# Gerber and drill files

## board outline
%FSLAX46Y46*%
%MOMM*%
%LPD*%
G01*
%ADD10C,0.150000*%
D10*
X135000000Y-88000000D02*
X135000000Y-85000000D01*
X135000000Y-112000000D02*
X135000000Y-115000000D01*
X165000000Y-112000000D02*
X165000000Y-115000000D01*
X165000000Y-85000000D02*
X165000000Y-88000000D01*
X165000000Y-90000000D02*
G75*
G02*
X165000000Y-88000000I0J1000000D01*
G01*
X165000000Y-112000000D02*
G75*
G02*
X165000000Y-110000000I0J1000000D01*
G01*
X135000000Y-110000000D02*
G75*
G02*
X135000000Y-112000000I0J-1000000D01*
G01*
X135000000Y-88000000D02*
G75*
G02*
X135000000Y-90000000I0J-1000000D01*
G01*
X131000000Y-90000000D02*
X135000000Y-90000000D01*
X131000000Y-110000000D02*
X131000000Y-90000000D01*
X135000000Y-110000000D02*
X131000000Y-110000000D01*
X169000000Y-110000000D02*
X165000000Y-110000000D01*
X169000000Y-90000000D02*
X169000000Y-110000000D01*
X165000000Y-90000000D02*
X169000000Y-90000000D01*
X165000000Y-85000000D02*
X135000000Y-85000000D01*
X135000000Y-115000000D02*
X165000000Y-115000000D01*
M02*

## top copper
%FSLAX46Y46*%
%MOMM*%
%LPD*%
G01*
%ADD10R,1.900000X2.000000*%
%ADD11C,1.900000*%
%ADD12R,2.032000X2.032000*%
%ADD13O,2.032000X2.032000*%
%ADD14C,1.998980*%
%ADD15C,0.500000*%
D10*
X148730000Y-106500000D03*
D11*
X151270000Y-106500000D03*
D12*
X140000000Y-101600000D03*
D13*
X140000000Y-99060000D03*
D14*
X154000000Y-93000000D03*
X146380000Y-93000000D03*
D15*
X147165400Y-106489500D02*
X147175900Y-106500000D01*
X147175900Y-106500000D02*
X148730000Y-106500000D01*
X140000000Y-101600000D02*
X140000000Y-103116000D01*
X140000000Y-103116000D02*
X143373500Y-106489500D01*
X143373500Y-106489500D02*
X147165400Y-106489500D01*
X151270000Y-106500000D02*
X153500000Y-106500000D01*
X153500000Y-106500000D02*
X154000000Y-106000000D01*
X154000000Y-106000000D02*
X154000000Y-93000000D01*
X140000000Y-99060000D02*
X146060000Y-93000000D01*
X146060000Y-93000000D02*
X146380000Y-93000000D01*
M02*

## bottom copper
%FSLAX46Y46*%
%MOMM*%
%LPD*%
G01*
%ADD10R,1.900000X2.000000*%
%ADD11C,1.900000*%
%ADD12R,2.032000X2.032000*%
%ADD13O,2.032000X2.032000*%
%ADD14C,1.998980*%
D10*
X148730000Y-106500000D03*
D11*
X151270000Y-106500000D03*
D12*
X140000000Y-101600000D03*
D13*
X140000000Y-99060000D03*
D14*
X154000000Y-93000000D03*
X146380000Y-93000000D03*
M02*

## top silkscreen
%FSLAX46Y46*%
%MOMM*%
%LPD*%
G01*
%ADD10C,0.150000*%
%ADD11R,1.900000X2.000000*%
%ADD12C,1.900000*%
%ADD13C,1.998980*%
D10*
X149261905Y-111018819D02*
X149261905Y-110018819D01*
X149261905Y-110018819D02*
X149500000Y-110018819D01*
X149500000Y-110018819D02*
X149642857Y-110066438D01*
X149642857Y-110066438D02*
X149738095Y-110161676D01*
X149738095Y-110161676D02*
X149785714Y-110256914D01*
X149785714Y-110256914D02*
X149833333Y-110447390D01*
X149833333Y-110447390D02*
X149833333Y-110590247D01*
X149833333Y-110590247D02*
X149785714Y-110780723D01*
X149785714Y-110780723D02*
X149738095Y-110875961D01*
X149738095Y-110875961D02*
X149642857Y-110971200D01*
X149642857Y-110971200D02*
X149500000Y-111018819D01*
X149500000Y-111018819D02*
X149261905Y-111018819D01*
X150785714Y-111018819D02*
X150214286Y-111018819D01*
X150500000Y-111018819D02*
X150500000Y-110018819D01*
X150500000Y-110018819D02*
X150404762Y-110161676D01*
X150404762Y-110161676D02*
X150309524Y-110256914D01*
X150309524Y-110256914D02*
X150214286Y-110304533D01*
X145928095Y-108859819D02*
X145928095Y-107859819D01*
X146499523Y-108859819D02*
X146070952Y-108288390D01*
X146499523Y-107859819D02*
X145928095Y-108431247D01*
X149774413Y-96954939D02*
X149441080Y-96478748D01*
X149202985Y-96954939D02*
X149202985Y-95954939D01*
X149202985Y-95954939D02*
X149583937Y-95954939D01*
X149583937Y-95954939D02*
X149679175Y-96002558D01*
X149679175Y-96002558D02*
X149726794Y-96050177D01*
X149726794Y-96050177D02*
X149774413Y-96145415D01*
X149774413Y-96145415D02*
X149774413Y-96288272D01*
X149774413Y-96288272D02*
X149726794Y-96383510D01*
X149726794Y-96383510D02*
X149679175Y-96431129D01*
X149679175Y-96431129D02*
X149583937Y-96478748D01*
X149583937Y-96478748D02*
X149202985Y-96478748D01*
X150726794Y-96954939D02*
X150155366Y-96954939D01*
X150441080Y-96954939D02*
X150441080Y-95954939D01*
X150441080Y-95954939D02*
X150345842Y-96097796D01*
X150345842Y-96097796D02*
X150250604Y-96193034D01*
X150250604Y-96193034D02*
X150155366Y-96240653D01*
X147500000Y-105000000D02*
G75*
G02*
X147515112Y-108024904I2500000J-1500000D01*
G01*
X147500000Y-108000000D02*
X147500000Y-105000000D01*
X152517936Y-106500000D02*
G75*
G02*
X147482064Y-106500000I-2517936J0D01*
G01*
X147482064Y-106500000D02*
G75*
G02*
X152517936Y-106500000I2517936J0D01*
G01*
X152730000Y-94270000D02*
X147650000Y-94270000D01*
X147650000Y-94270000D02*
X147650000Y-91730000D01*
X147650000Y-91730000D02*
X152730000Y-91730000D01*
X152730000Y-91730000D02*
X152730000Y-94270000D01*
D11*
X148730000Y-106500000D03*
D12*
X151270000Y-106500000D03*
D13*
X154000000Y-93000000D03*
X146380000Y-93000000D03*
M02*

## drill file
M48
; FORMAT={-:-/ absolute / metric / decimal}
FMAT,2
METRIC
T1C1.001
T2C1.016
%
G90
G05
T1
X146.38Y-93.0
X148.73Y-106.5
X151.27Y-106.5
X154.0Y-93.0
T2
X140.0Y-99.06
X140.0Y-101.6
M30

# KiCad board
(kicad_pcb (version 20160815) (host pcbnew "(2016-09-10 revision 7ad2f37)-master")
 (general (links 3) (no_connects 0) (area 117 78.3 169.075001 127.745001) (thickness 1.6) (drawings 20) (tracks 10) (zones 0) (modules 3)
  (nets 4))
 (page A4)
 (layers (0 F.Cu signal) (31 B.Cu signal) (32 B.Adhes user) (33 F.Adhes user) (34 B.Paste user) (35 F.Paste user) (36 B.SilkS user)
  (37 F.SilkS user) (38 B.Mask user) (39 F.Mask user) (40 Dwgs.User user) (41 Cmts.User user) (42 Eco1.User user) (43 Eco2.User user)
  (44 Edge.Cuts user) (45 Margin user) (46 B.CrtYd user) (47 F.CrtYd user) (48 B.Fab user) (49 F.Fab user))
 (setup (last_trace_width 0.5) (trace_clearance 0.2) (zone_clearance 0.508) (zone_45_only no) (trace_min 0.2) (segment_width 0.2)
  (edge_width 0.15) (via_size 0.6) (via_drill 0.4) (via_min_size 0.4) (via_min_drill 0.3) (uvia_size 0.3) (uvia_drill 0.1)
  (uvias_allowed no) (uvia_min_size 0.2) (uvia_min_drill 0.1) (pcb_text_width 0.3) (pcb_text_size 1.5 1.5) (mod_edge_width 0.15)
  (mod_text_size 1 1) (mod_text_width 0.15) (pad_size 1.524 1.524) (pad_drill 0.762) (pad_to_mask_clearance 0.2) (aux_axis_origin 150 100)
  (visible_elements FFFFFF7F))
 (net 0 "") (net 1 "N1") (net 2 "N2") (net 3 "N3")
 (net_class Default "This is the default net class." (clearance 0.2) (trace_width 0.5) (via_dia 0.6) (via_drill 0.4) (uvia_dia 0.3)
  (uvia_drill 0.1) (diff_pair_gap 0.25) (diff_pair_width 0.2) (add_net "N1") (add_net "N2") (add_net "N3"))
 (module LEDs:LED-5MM (layer F.Cu) (at 150 106.5)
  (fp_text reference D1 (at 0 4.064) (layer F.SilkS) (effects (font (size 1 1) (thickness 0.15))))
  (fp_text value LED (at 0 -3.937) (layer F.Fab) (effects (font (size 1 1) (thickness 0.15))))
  (fp_arc (start 0 0) (end -2.5 -1.5) (angle 297.5) (layer F.SilkS) (width 0.15))
  (fp_line (start -2.5 1.5) (end -2.5 -1.5) (layer F.SilkS) (width 0.15))
  (fp_circle (center 0 0) (end -0.3 -2.5) (layer F.SilkS) (width 0.15))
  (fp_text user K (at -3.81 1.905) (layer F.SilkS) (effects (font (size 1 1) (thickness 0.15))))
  (pad 1 thru_hole rect (at -1.27 0 90) (size 2 1.9) (drill 1.00076) (layers *.Cu *.Mask F.SilkS) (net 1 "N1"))
  (pad 2 thru_hole circle (at 1.27 0) (size 1.9 1.9) (drill 1.00076) (layers *.Cu *.Mask F.SilkS) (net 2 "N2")))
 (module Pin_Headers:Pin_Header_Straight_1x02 (layer B.Cu) (at 140 101.6)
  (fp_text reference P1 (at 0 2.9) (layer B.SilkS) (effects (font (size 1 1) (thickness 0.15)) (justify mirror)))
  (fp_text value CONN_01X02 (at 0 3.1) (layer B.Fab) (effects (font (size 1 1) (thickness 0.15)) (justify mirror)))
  (pad 1 thru_hole rect (at 0 0) (size 2.032 2.032) (drill 1.016) (layers *.Cu *.Mask B.SilkS) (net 1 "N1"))
  (pad 2 thru_hole oval (at 0 -2.54) (size 2.032 2.032) (drill 1.016) (layers *.Cu *.Mask B.SilkS) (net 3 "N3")))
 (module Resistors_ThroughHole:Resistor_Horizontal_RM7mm (layer F.Cu) (at 154 93 180)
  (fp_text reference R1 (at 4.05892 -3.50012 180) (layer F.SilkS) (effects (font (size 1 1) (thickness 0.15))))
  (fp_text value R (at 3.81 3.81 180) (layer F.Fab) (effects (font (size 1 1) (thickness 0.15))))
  (fp_line (start 1.27 -1.27) (end 6.35 -1.27) (layer F.SilkS) (width 0.15))
  (fp_line (start 6.35 -1.27) (end 6.35 1.27) (layer F.SilkS) (width 0.15))
  (fp_line (start 6.35 1.27) (end 1.27 1.27) (layer F.SilkS) (width 0.15))
  (fp_line (start 1.27 1.27) (end 1.27 -1.27) (layer F.SilkS) (width 0.15))
  (pad 1 thru_hole circle (at 0 0 180) (size 1.99898 1.99898) (drill 1.00076) (layers *.Cu *.SilkS *.Mask) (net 2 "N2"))
  (pad 2 thru_hole circle (at 7.62 0 180) (size 1.99898 1.99898) (drill 1.00076) (layers *.Cu *.SilkS *.Mask) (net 3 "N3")))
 (gr_line (start 135 88) (end 135 85) (layer Edge.Cuts) (width 0.15))
 (gr_line (start 135 112) (end 135 115) (layer Edge.Cuts) (width 0.15))
 (gr_line (start 165 112) (end 165 115) (layer Edge.Cuts) (width 0.15))
 (gr_line (start 165 85) (end 165 88) (layer Edge.Cuts) (width 0.15))
 (gr_arc (start 165 89) (end 165 90) (angle 180) (layer Edge.Cuts) (width 0.15))
 (gr_arc (start 165 111) (end 165 112) (angle 180) (layer Edge.Cuts) (width 0.15))
 (gr_arc (start 135 111) (end 135 110) (angle 180) (layer Edge.Cuts) (width 0.15))
 (gr_arc (start 135 89) (end 135 88) (angle 180) (layer Edge.Cuts) (width 0.15))
 (gr_line (start 131 90) (end 135 90) (layer Edge.Cuts) (width 0.15))
 (gr_line (start 131 110) (end 131 90) (layer Edge.Cuts) (width 0.15))
 (gr_line (start 135 110) (end 131 110) (layer Edge.Cuts) (width 0.15))
 (gr_line (start 169 110) (end 165 110) (layer Edge.Cuts) (width 0.15))
 (gr_line (start 169 90) (end 169 110) (layer Edge.Cuts) (width 0.15))
 (gr_line (start 165 90) (end 169 90) (layer Edge.Cuts) (width 0.15))
 (gr_line (start 165 85) (end 135 85) (layer Edge.Cuts) (width 0.15))
 (gr_line (start 135 115) (end 165 115) (layer Edge.Cuts) (width 0.15))
 (segment (start 147.1654 106.4895) (end 147.1759 106.5) (width 0.5) (layer F.Cu) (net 1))
 (segment (start 147.1759 106.5) (end 148.73 106.5) (width 0.5) (layer F.Cu) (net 1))
 (segment (start 140 101.6) (end 140 103.116) (width 0.5) (layer F.Cu) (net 1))
 (segment (start 140 103.116) (end 143.3735 106.4895) (width 0.5) (layer F.Cu) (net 1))
 (segment (start 143.3735 106.4895) (end 147.1654 106.4895) (width 0.5) (layer F.Cu) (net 1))
 (segment (start 151.27 106.5) (end 153.5 106.5) (width 0.5) (layer F.Cu) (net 2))
 (segment (start 153.5 106.5) (end 154 106) (width 0.5) (layer F.Cu) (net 2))
 (segment (start 154 106) (end 154 93) (width 0.5) (layer F.Cu) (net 2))
 (segment (start 140 99.06) (end 146.06 93) (width 0.5) (layer F.Cu) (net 3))
 (segment (start 146.06 93) (end 146.38 93) (width 0.5) (layer F.Cu) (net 3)))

